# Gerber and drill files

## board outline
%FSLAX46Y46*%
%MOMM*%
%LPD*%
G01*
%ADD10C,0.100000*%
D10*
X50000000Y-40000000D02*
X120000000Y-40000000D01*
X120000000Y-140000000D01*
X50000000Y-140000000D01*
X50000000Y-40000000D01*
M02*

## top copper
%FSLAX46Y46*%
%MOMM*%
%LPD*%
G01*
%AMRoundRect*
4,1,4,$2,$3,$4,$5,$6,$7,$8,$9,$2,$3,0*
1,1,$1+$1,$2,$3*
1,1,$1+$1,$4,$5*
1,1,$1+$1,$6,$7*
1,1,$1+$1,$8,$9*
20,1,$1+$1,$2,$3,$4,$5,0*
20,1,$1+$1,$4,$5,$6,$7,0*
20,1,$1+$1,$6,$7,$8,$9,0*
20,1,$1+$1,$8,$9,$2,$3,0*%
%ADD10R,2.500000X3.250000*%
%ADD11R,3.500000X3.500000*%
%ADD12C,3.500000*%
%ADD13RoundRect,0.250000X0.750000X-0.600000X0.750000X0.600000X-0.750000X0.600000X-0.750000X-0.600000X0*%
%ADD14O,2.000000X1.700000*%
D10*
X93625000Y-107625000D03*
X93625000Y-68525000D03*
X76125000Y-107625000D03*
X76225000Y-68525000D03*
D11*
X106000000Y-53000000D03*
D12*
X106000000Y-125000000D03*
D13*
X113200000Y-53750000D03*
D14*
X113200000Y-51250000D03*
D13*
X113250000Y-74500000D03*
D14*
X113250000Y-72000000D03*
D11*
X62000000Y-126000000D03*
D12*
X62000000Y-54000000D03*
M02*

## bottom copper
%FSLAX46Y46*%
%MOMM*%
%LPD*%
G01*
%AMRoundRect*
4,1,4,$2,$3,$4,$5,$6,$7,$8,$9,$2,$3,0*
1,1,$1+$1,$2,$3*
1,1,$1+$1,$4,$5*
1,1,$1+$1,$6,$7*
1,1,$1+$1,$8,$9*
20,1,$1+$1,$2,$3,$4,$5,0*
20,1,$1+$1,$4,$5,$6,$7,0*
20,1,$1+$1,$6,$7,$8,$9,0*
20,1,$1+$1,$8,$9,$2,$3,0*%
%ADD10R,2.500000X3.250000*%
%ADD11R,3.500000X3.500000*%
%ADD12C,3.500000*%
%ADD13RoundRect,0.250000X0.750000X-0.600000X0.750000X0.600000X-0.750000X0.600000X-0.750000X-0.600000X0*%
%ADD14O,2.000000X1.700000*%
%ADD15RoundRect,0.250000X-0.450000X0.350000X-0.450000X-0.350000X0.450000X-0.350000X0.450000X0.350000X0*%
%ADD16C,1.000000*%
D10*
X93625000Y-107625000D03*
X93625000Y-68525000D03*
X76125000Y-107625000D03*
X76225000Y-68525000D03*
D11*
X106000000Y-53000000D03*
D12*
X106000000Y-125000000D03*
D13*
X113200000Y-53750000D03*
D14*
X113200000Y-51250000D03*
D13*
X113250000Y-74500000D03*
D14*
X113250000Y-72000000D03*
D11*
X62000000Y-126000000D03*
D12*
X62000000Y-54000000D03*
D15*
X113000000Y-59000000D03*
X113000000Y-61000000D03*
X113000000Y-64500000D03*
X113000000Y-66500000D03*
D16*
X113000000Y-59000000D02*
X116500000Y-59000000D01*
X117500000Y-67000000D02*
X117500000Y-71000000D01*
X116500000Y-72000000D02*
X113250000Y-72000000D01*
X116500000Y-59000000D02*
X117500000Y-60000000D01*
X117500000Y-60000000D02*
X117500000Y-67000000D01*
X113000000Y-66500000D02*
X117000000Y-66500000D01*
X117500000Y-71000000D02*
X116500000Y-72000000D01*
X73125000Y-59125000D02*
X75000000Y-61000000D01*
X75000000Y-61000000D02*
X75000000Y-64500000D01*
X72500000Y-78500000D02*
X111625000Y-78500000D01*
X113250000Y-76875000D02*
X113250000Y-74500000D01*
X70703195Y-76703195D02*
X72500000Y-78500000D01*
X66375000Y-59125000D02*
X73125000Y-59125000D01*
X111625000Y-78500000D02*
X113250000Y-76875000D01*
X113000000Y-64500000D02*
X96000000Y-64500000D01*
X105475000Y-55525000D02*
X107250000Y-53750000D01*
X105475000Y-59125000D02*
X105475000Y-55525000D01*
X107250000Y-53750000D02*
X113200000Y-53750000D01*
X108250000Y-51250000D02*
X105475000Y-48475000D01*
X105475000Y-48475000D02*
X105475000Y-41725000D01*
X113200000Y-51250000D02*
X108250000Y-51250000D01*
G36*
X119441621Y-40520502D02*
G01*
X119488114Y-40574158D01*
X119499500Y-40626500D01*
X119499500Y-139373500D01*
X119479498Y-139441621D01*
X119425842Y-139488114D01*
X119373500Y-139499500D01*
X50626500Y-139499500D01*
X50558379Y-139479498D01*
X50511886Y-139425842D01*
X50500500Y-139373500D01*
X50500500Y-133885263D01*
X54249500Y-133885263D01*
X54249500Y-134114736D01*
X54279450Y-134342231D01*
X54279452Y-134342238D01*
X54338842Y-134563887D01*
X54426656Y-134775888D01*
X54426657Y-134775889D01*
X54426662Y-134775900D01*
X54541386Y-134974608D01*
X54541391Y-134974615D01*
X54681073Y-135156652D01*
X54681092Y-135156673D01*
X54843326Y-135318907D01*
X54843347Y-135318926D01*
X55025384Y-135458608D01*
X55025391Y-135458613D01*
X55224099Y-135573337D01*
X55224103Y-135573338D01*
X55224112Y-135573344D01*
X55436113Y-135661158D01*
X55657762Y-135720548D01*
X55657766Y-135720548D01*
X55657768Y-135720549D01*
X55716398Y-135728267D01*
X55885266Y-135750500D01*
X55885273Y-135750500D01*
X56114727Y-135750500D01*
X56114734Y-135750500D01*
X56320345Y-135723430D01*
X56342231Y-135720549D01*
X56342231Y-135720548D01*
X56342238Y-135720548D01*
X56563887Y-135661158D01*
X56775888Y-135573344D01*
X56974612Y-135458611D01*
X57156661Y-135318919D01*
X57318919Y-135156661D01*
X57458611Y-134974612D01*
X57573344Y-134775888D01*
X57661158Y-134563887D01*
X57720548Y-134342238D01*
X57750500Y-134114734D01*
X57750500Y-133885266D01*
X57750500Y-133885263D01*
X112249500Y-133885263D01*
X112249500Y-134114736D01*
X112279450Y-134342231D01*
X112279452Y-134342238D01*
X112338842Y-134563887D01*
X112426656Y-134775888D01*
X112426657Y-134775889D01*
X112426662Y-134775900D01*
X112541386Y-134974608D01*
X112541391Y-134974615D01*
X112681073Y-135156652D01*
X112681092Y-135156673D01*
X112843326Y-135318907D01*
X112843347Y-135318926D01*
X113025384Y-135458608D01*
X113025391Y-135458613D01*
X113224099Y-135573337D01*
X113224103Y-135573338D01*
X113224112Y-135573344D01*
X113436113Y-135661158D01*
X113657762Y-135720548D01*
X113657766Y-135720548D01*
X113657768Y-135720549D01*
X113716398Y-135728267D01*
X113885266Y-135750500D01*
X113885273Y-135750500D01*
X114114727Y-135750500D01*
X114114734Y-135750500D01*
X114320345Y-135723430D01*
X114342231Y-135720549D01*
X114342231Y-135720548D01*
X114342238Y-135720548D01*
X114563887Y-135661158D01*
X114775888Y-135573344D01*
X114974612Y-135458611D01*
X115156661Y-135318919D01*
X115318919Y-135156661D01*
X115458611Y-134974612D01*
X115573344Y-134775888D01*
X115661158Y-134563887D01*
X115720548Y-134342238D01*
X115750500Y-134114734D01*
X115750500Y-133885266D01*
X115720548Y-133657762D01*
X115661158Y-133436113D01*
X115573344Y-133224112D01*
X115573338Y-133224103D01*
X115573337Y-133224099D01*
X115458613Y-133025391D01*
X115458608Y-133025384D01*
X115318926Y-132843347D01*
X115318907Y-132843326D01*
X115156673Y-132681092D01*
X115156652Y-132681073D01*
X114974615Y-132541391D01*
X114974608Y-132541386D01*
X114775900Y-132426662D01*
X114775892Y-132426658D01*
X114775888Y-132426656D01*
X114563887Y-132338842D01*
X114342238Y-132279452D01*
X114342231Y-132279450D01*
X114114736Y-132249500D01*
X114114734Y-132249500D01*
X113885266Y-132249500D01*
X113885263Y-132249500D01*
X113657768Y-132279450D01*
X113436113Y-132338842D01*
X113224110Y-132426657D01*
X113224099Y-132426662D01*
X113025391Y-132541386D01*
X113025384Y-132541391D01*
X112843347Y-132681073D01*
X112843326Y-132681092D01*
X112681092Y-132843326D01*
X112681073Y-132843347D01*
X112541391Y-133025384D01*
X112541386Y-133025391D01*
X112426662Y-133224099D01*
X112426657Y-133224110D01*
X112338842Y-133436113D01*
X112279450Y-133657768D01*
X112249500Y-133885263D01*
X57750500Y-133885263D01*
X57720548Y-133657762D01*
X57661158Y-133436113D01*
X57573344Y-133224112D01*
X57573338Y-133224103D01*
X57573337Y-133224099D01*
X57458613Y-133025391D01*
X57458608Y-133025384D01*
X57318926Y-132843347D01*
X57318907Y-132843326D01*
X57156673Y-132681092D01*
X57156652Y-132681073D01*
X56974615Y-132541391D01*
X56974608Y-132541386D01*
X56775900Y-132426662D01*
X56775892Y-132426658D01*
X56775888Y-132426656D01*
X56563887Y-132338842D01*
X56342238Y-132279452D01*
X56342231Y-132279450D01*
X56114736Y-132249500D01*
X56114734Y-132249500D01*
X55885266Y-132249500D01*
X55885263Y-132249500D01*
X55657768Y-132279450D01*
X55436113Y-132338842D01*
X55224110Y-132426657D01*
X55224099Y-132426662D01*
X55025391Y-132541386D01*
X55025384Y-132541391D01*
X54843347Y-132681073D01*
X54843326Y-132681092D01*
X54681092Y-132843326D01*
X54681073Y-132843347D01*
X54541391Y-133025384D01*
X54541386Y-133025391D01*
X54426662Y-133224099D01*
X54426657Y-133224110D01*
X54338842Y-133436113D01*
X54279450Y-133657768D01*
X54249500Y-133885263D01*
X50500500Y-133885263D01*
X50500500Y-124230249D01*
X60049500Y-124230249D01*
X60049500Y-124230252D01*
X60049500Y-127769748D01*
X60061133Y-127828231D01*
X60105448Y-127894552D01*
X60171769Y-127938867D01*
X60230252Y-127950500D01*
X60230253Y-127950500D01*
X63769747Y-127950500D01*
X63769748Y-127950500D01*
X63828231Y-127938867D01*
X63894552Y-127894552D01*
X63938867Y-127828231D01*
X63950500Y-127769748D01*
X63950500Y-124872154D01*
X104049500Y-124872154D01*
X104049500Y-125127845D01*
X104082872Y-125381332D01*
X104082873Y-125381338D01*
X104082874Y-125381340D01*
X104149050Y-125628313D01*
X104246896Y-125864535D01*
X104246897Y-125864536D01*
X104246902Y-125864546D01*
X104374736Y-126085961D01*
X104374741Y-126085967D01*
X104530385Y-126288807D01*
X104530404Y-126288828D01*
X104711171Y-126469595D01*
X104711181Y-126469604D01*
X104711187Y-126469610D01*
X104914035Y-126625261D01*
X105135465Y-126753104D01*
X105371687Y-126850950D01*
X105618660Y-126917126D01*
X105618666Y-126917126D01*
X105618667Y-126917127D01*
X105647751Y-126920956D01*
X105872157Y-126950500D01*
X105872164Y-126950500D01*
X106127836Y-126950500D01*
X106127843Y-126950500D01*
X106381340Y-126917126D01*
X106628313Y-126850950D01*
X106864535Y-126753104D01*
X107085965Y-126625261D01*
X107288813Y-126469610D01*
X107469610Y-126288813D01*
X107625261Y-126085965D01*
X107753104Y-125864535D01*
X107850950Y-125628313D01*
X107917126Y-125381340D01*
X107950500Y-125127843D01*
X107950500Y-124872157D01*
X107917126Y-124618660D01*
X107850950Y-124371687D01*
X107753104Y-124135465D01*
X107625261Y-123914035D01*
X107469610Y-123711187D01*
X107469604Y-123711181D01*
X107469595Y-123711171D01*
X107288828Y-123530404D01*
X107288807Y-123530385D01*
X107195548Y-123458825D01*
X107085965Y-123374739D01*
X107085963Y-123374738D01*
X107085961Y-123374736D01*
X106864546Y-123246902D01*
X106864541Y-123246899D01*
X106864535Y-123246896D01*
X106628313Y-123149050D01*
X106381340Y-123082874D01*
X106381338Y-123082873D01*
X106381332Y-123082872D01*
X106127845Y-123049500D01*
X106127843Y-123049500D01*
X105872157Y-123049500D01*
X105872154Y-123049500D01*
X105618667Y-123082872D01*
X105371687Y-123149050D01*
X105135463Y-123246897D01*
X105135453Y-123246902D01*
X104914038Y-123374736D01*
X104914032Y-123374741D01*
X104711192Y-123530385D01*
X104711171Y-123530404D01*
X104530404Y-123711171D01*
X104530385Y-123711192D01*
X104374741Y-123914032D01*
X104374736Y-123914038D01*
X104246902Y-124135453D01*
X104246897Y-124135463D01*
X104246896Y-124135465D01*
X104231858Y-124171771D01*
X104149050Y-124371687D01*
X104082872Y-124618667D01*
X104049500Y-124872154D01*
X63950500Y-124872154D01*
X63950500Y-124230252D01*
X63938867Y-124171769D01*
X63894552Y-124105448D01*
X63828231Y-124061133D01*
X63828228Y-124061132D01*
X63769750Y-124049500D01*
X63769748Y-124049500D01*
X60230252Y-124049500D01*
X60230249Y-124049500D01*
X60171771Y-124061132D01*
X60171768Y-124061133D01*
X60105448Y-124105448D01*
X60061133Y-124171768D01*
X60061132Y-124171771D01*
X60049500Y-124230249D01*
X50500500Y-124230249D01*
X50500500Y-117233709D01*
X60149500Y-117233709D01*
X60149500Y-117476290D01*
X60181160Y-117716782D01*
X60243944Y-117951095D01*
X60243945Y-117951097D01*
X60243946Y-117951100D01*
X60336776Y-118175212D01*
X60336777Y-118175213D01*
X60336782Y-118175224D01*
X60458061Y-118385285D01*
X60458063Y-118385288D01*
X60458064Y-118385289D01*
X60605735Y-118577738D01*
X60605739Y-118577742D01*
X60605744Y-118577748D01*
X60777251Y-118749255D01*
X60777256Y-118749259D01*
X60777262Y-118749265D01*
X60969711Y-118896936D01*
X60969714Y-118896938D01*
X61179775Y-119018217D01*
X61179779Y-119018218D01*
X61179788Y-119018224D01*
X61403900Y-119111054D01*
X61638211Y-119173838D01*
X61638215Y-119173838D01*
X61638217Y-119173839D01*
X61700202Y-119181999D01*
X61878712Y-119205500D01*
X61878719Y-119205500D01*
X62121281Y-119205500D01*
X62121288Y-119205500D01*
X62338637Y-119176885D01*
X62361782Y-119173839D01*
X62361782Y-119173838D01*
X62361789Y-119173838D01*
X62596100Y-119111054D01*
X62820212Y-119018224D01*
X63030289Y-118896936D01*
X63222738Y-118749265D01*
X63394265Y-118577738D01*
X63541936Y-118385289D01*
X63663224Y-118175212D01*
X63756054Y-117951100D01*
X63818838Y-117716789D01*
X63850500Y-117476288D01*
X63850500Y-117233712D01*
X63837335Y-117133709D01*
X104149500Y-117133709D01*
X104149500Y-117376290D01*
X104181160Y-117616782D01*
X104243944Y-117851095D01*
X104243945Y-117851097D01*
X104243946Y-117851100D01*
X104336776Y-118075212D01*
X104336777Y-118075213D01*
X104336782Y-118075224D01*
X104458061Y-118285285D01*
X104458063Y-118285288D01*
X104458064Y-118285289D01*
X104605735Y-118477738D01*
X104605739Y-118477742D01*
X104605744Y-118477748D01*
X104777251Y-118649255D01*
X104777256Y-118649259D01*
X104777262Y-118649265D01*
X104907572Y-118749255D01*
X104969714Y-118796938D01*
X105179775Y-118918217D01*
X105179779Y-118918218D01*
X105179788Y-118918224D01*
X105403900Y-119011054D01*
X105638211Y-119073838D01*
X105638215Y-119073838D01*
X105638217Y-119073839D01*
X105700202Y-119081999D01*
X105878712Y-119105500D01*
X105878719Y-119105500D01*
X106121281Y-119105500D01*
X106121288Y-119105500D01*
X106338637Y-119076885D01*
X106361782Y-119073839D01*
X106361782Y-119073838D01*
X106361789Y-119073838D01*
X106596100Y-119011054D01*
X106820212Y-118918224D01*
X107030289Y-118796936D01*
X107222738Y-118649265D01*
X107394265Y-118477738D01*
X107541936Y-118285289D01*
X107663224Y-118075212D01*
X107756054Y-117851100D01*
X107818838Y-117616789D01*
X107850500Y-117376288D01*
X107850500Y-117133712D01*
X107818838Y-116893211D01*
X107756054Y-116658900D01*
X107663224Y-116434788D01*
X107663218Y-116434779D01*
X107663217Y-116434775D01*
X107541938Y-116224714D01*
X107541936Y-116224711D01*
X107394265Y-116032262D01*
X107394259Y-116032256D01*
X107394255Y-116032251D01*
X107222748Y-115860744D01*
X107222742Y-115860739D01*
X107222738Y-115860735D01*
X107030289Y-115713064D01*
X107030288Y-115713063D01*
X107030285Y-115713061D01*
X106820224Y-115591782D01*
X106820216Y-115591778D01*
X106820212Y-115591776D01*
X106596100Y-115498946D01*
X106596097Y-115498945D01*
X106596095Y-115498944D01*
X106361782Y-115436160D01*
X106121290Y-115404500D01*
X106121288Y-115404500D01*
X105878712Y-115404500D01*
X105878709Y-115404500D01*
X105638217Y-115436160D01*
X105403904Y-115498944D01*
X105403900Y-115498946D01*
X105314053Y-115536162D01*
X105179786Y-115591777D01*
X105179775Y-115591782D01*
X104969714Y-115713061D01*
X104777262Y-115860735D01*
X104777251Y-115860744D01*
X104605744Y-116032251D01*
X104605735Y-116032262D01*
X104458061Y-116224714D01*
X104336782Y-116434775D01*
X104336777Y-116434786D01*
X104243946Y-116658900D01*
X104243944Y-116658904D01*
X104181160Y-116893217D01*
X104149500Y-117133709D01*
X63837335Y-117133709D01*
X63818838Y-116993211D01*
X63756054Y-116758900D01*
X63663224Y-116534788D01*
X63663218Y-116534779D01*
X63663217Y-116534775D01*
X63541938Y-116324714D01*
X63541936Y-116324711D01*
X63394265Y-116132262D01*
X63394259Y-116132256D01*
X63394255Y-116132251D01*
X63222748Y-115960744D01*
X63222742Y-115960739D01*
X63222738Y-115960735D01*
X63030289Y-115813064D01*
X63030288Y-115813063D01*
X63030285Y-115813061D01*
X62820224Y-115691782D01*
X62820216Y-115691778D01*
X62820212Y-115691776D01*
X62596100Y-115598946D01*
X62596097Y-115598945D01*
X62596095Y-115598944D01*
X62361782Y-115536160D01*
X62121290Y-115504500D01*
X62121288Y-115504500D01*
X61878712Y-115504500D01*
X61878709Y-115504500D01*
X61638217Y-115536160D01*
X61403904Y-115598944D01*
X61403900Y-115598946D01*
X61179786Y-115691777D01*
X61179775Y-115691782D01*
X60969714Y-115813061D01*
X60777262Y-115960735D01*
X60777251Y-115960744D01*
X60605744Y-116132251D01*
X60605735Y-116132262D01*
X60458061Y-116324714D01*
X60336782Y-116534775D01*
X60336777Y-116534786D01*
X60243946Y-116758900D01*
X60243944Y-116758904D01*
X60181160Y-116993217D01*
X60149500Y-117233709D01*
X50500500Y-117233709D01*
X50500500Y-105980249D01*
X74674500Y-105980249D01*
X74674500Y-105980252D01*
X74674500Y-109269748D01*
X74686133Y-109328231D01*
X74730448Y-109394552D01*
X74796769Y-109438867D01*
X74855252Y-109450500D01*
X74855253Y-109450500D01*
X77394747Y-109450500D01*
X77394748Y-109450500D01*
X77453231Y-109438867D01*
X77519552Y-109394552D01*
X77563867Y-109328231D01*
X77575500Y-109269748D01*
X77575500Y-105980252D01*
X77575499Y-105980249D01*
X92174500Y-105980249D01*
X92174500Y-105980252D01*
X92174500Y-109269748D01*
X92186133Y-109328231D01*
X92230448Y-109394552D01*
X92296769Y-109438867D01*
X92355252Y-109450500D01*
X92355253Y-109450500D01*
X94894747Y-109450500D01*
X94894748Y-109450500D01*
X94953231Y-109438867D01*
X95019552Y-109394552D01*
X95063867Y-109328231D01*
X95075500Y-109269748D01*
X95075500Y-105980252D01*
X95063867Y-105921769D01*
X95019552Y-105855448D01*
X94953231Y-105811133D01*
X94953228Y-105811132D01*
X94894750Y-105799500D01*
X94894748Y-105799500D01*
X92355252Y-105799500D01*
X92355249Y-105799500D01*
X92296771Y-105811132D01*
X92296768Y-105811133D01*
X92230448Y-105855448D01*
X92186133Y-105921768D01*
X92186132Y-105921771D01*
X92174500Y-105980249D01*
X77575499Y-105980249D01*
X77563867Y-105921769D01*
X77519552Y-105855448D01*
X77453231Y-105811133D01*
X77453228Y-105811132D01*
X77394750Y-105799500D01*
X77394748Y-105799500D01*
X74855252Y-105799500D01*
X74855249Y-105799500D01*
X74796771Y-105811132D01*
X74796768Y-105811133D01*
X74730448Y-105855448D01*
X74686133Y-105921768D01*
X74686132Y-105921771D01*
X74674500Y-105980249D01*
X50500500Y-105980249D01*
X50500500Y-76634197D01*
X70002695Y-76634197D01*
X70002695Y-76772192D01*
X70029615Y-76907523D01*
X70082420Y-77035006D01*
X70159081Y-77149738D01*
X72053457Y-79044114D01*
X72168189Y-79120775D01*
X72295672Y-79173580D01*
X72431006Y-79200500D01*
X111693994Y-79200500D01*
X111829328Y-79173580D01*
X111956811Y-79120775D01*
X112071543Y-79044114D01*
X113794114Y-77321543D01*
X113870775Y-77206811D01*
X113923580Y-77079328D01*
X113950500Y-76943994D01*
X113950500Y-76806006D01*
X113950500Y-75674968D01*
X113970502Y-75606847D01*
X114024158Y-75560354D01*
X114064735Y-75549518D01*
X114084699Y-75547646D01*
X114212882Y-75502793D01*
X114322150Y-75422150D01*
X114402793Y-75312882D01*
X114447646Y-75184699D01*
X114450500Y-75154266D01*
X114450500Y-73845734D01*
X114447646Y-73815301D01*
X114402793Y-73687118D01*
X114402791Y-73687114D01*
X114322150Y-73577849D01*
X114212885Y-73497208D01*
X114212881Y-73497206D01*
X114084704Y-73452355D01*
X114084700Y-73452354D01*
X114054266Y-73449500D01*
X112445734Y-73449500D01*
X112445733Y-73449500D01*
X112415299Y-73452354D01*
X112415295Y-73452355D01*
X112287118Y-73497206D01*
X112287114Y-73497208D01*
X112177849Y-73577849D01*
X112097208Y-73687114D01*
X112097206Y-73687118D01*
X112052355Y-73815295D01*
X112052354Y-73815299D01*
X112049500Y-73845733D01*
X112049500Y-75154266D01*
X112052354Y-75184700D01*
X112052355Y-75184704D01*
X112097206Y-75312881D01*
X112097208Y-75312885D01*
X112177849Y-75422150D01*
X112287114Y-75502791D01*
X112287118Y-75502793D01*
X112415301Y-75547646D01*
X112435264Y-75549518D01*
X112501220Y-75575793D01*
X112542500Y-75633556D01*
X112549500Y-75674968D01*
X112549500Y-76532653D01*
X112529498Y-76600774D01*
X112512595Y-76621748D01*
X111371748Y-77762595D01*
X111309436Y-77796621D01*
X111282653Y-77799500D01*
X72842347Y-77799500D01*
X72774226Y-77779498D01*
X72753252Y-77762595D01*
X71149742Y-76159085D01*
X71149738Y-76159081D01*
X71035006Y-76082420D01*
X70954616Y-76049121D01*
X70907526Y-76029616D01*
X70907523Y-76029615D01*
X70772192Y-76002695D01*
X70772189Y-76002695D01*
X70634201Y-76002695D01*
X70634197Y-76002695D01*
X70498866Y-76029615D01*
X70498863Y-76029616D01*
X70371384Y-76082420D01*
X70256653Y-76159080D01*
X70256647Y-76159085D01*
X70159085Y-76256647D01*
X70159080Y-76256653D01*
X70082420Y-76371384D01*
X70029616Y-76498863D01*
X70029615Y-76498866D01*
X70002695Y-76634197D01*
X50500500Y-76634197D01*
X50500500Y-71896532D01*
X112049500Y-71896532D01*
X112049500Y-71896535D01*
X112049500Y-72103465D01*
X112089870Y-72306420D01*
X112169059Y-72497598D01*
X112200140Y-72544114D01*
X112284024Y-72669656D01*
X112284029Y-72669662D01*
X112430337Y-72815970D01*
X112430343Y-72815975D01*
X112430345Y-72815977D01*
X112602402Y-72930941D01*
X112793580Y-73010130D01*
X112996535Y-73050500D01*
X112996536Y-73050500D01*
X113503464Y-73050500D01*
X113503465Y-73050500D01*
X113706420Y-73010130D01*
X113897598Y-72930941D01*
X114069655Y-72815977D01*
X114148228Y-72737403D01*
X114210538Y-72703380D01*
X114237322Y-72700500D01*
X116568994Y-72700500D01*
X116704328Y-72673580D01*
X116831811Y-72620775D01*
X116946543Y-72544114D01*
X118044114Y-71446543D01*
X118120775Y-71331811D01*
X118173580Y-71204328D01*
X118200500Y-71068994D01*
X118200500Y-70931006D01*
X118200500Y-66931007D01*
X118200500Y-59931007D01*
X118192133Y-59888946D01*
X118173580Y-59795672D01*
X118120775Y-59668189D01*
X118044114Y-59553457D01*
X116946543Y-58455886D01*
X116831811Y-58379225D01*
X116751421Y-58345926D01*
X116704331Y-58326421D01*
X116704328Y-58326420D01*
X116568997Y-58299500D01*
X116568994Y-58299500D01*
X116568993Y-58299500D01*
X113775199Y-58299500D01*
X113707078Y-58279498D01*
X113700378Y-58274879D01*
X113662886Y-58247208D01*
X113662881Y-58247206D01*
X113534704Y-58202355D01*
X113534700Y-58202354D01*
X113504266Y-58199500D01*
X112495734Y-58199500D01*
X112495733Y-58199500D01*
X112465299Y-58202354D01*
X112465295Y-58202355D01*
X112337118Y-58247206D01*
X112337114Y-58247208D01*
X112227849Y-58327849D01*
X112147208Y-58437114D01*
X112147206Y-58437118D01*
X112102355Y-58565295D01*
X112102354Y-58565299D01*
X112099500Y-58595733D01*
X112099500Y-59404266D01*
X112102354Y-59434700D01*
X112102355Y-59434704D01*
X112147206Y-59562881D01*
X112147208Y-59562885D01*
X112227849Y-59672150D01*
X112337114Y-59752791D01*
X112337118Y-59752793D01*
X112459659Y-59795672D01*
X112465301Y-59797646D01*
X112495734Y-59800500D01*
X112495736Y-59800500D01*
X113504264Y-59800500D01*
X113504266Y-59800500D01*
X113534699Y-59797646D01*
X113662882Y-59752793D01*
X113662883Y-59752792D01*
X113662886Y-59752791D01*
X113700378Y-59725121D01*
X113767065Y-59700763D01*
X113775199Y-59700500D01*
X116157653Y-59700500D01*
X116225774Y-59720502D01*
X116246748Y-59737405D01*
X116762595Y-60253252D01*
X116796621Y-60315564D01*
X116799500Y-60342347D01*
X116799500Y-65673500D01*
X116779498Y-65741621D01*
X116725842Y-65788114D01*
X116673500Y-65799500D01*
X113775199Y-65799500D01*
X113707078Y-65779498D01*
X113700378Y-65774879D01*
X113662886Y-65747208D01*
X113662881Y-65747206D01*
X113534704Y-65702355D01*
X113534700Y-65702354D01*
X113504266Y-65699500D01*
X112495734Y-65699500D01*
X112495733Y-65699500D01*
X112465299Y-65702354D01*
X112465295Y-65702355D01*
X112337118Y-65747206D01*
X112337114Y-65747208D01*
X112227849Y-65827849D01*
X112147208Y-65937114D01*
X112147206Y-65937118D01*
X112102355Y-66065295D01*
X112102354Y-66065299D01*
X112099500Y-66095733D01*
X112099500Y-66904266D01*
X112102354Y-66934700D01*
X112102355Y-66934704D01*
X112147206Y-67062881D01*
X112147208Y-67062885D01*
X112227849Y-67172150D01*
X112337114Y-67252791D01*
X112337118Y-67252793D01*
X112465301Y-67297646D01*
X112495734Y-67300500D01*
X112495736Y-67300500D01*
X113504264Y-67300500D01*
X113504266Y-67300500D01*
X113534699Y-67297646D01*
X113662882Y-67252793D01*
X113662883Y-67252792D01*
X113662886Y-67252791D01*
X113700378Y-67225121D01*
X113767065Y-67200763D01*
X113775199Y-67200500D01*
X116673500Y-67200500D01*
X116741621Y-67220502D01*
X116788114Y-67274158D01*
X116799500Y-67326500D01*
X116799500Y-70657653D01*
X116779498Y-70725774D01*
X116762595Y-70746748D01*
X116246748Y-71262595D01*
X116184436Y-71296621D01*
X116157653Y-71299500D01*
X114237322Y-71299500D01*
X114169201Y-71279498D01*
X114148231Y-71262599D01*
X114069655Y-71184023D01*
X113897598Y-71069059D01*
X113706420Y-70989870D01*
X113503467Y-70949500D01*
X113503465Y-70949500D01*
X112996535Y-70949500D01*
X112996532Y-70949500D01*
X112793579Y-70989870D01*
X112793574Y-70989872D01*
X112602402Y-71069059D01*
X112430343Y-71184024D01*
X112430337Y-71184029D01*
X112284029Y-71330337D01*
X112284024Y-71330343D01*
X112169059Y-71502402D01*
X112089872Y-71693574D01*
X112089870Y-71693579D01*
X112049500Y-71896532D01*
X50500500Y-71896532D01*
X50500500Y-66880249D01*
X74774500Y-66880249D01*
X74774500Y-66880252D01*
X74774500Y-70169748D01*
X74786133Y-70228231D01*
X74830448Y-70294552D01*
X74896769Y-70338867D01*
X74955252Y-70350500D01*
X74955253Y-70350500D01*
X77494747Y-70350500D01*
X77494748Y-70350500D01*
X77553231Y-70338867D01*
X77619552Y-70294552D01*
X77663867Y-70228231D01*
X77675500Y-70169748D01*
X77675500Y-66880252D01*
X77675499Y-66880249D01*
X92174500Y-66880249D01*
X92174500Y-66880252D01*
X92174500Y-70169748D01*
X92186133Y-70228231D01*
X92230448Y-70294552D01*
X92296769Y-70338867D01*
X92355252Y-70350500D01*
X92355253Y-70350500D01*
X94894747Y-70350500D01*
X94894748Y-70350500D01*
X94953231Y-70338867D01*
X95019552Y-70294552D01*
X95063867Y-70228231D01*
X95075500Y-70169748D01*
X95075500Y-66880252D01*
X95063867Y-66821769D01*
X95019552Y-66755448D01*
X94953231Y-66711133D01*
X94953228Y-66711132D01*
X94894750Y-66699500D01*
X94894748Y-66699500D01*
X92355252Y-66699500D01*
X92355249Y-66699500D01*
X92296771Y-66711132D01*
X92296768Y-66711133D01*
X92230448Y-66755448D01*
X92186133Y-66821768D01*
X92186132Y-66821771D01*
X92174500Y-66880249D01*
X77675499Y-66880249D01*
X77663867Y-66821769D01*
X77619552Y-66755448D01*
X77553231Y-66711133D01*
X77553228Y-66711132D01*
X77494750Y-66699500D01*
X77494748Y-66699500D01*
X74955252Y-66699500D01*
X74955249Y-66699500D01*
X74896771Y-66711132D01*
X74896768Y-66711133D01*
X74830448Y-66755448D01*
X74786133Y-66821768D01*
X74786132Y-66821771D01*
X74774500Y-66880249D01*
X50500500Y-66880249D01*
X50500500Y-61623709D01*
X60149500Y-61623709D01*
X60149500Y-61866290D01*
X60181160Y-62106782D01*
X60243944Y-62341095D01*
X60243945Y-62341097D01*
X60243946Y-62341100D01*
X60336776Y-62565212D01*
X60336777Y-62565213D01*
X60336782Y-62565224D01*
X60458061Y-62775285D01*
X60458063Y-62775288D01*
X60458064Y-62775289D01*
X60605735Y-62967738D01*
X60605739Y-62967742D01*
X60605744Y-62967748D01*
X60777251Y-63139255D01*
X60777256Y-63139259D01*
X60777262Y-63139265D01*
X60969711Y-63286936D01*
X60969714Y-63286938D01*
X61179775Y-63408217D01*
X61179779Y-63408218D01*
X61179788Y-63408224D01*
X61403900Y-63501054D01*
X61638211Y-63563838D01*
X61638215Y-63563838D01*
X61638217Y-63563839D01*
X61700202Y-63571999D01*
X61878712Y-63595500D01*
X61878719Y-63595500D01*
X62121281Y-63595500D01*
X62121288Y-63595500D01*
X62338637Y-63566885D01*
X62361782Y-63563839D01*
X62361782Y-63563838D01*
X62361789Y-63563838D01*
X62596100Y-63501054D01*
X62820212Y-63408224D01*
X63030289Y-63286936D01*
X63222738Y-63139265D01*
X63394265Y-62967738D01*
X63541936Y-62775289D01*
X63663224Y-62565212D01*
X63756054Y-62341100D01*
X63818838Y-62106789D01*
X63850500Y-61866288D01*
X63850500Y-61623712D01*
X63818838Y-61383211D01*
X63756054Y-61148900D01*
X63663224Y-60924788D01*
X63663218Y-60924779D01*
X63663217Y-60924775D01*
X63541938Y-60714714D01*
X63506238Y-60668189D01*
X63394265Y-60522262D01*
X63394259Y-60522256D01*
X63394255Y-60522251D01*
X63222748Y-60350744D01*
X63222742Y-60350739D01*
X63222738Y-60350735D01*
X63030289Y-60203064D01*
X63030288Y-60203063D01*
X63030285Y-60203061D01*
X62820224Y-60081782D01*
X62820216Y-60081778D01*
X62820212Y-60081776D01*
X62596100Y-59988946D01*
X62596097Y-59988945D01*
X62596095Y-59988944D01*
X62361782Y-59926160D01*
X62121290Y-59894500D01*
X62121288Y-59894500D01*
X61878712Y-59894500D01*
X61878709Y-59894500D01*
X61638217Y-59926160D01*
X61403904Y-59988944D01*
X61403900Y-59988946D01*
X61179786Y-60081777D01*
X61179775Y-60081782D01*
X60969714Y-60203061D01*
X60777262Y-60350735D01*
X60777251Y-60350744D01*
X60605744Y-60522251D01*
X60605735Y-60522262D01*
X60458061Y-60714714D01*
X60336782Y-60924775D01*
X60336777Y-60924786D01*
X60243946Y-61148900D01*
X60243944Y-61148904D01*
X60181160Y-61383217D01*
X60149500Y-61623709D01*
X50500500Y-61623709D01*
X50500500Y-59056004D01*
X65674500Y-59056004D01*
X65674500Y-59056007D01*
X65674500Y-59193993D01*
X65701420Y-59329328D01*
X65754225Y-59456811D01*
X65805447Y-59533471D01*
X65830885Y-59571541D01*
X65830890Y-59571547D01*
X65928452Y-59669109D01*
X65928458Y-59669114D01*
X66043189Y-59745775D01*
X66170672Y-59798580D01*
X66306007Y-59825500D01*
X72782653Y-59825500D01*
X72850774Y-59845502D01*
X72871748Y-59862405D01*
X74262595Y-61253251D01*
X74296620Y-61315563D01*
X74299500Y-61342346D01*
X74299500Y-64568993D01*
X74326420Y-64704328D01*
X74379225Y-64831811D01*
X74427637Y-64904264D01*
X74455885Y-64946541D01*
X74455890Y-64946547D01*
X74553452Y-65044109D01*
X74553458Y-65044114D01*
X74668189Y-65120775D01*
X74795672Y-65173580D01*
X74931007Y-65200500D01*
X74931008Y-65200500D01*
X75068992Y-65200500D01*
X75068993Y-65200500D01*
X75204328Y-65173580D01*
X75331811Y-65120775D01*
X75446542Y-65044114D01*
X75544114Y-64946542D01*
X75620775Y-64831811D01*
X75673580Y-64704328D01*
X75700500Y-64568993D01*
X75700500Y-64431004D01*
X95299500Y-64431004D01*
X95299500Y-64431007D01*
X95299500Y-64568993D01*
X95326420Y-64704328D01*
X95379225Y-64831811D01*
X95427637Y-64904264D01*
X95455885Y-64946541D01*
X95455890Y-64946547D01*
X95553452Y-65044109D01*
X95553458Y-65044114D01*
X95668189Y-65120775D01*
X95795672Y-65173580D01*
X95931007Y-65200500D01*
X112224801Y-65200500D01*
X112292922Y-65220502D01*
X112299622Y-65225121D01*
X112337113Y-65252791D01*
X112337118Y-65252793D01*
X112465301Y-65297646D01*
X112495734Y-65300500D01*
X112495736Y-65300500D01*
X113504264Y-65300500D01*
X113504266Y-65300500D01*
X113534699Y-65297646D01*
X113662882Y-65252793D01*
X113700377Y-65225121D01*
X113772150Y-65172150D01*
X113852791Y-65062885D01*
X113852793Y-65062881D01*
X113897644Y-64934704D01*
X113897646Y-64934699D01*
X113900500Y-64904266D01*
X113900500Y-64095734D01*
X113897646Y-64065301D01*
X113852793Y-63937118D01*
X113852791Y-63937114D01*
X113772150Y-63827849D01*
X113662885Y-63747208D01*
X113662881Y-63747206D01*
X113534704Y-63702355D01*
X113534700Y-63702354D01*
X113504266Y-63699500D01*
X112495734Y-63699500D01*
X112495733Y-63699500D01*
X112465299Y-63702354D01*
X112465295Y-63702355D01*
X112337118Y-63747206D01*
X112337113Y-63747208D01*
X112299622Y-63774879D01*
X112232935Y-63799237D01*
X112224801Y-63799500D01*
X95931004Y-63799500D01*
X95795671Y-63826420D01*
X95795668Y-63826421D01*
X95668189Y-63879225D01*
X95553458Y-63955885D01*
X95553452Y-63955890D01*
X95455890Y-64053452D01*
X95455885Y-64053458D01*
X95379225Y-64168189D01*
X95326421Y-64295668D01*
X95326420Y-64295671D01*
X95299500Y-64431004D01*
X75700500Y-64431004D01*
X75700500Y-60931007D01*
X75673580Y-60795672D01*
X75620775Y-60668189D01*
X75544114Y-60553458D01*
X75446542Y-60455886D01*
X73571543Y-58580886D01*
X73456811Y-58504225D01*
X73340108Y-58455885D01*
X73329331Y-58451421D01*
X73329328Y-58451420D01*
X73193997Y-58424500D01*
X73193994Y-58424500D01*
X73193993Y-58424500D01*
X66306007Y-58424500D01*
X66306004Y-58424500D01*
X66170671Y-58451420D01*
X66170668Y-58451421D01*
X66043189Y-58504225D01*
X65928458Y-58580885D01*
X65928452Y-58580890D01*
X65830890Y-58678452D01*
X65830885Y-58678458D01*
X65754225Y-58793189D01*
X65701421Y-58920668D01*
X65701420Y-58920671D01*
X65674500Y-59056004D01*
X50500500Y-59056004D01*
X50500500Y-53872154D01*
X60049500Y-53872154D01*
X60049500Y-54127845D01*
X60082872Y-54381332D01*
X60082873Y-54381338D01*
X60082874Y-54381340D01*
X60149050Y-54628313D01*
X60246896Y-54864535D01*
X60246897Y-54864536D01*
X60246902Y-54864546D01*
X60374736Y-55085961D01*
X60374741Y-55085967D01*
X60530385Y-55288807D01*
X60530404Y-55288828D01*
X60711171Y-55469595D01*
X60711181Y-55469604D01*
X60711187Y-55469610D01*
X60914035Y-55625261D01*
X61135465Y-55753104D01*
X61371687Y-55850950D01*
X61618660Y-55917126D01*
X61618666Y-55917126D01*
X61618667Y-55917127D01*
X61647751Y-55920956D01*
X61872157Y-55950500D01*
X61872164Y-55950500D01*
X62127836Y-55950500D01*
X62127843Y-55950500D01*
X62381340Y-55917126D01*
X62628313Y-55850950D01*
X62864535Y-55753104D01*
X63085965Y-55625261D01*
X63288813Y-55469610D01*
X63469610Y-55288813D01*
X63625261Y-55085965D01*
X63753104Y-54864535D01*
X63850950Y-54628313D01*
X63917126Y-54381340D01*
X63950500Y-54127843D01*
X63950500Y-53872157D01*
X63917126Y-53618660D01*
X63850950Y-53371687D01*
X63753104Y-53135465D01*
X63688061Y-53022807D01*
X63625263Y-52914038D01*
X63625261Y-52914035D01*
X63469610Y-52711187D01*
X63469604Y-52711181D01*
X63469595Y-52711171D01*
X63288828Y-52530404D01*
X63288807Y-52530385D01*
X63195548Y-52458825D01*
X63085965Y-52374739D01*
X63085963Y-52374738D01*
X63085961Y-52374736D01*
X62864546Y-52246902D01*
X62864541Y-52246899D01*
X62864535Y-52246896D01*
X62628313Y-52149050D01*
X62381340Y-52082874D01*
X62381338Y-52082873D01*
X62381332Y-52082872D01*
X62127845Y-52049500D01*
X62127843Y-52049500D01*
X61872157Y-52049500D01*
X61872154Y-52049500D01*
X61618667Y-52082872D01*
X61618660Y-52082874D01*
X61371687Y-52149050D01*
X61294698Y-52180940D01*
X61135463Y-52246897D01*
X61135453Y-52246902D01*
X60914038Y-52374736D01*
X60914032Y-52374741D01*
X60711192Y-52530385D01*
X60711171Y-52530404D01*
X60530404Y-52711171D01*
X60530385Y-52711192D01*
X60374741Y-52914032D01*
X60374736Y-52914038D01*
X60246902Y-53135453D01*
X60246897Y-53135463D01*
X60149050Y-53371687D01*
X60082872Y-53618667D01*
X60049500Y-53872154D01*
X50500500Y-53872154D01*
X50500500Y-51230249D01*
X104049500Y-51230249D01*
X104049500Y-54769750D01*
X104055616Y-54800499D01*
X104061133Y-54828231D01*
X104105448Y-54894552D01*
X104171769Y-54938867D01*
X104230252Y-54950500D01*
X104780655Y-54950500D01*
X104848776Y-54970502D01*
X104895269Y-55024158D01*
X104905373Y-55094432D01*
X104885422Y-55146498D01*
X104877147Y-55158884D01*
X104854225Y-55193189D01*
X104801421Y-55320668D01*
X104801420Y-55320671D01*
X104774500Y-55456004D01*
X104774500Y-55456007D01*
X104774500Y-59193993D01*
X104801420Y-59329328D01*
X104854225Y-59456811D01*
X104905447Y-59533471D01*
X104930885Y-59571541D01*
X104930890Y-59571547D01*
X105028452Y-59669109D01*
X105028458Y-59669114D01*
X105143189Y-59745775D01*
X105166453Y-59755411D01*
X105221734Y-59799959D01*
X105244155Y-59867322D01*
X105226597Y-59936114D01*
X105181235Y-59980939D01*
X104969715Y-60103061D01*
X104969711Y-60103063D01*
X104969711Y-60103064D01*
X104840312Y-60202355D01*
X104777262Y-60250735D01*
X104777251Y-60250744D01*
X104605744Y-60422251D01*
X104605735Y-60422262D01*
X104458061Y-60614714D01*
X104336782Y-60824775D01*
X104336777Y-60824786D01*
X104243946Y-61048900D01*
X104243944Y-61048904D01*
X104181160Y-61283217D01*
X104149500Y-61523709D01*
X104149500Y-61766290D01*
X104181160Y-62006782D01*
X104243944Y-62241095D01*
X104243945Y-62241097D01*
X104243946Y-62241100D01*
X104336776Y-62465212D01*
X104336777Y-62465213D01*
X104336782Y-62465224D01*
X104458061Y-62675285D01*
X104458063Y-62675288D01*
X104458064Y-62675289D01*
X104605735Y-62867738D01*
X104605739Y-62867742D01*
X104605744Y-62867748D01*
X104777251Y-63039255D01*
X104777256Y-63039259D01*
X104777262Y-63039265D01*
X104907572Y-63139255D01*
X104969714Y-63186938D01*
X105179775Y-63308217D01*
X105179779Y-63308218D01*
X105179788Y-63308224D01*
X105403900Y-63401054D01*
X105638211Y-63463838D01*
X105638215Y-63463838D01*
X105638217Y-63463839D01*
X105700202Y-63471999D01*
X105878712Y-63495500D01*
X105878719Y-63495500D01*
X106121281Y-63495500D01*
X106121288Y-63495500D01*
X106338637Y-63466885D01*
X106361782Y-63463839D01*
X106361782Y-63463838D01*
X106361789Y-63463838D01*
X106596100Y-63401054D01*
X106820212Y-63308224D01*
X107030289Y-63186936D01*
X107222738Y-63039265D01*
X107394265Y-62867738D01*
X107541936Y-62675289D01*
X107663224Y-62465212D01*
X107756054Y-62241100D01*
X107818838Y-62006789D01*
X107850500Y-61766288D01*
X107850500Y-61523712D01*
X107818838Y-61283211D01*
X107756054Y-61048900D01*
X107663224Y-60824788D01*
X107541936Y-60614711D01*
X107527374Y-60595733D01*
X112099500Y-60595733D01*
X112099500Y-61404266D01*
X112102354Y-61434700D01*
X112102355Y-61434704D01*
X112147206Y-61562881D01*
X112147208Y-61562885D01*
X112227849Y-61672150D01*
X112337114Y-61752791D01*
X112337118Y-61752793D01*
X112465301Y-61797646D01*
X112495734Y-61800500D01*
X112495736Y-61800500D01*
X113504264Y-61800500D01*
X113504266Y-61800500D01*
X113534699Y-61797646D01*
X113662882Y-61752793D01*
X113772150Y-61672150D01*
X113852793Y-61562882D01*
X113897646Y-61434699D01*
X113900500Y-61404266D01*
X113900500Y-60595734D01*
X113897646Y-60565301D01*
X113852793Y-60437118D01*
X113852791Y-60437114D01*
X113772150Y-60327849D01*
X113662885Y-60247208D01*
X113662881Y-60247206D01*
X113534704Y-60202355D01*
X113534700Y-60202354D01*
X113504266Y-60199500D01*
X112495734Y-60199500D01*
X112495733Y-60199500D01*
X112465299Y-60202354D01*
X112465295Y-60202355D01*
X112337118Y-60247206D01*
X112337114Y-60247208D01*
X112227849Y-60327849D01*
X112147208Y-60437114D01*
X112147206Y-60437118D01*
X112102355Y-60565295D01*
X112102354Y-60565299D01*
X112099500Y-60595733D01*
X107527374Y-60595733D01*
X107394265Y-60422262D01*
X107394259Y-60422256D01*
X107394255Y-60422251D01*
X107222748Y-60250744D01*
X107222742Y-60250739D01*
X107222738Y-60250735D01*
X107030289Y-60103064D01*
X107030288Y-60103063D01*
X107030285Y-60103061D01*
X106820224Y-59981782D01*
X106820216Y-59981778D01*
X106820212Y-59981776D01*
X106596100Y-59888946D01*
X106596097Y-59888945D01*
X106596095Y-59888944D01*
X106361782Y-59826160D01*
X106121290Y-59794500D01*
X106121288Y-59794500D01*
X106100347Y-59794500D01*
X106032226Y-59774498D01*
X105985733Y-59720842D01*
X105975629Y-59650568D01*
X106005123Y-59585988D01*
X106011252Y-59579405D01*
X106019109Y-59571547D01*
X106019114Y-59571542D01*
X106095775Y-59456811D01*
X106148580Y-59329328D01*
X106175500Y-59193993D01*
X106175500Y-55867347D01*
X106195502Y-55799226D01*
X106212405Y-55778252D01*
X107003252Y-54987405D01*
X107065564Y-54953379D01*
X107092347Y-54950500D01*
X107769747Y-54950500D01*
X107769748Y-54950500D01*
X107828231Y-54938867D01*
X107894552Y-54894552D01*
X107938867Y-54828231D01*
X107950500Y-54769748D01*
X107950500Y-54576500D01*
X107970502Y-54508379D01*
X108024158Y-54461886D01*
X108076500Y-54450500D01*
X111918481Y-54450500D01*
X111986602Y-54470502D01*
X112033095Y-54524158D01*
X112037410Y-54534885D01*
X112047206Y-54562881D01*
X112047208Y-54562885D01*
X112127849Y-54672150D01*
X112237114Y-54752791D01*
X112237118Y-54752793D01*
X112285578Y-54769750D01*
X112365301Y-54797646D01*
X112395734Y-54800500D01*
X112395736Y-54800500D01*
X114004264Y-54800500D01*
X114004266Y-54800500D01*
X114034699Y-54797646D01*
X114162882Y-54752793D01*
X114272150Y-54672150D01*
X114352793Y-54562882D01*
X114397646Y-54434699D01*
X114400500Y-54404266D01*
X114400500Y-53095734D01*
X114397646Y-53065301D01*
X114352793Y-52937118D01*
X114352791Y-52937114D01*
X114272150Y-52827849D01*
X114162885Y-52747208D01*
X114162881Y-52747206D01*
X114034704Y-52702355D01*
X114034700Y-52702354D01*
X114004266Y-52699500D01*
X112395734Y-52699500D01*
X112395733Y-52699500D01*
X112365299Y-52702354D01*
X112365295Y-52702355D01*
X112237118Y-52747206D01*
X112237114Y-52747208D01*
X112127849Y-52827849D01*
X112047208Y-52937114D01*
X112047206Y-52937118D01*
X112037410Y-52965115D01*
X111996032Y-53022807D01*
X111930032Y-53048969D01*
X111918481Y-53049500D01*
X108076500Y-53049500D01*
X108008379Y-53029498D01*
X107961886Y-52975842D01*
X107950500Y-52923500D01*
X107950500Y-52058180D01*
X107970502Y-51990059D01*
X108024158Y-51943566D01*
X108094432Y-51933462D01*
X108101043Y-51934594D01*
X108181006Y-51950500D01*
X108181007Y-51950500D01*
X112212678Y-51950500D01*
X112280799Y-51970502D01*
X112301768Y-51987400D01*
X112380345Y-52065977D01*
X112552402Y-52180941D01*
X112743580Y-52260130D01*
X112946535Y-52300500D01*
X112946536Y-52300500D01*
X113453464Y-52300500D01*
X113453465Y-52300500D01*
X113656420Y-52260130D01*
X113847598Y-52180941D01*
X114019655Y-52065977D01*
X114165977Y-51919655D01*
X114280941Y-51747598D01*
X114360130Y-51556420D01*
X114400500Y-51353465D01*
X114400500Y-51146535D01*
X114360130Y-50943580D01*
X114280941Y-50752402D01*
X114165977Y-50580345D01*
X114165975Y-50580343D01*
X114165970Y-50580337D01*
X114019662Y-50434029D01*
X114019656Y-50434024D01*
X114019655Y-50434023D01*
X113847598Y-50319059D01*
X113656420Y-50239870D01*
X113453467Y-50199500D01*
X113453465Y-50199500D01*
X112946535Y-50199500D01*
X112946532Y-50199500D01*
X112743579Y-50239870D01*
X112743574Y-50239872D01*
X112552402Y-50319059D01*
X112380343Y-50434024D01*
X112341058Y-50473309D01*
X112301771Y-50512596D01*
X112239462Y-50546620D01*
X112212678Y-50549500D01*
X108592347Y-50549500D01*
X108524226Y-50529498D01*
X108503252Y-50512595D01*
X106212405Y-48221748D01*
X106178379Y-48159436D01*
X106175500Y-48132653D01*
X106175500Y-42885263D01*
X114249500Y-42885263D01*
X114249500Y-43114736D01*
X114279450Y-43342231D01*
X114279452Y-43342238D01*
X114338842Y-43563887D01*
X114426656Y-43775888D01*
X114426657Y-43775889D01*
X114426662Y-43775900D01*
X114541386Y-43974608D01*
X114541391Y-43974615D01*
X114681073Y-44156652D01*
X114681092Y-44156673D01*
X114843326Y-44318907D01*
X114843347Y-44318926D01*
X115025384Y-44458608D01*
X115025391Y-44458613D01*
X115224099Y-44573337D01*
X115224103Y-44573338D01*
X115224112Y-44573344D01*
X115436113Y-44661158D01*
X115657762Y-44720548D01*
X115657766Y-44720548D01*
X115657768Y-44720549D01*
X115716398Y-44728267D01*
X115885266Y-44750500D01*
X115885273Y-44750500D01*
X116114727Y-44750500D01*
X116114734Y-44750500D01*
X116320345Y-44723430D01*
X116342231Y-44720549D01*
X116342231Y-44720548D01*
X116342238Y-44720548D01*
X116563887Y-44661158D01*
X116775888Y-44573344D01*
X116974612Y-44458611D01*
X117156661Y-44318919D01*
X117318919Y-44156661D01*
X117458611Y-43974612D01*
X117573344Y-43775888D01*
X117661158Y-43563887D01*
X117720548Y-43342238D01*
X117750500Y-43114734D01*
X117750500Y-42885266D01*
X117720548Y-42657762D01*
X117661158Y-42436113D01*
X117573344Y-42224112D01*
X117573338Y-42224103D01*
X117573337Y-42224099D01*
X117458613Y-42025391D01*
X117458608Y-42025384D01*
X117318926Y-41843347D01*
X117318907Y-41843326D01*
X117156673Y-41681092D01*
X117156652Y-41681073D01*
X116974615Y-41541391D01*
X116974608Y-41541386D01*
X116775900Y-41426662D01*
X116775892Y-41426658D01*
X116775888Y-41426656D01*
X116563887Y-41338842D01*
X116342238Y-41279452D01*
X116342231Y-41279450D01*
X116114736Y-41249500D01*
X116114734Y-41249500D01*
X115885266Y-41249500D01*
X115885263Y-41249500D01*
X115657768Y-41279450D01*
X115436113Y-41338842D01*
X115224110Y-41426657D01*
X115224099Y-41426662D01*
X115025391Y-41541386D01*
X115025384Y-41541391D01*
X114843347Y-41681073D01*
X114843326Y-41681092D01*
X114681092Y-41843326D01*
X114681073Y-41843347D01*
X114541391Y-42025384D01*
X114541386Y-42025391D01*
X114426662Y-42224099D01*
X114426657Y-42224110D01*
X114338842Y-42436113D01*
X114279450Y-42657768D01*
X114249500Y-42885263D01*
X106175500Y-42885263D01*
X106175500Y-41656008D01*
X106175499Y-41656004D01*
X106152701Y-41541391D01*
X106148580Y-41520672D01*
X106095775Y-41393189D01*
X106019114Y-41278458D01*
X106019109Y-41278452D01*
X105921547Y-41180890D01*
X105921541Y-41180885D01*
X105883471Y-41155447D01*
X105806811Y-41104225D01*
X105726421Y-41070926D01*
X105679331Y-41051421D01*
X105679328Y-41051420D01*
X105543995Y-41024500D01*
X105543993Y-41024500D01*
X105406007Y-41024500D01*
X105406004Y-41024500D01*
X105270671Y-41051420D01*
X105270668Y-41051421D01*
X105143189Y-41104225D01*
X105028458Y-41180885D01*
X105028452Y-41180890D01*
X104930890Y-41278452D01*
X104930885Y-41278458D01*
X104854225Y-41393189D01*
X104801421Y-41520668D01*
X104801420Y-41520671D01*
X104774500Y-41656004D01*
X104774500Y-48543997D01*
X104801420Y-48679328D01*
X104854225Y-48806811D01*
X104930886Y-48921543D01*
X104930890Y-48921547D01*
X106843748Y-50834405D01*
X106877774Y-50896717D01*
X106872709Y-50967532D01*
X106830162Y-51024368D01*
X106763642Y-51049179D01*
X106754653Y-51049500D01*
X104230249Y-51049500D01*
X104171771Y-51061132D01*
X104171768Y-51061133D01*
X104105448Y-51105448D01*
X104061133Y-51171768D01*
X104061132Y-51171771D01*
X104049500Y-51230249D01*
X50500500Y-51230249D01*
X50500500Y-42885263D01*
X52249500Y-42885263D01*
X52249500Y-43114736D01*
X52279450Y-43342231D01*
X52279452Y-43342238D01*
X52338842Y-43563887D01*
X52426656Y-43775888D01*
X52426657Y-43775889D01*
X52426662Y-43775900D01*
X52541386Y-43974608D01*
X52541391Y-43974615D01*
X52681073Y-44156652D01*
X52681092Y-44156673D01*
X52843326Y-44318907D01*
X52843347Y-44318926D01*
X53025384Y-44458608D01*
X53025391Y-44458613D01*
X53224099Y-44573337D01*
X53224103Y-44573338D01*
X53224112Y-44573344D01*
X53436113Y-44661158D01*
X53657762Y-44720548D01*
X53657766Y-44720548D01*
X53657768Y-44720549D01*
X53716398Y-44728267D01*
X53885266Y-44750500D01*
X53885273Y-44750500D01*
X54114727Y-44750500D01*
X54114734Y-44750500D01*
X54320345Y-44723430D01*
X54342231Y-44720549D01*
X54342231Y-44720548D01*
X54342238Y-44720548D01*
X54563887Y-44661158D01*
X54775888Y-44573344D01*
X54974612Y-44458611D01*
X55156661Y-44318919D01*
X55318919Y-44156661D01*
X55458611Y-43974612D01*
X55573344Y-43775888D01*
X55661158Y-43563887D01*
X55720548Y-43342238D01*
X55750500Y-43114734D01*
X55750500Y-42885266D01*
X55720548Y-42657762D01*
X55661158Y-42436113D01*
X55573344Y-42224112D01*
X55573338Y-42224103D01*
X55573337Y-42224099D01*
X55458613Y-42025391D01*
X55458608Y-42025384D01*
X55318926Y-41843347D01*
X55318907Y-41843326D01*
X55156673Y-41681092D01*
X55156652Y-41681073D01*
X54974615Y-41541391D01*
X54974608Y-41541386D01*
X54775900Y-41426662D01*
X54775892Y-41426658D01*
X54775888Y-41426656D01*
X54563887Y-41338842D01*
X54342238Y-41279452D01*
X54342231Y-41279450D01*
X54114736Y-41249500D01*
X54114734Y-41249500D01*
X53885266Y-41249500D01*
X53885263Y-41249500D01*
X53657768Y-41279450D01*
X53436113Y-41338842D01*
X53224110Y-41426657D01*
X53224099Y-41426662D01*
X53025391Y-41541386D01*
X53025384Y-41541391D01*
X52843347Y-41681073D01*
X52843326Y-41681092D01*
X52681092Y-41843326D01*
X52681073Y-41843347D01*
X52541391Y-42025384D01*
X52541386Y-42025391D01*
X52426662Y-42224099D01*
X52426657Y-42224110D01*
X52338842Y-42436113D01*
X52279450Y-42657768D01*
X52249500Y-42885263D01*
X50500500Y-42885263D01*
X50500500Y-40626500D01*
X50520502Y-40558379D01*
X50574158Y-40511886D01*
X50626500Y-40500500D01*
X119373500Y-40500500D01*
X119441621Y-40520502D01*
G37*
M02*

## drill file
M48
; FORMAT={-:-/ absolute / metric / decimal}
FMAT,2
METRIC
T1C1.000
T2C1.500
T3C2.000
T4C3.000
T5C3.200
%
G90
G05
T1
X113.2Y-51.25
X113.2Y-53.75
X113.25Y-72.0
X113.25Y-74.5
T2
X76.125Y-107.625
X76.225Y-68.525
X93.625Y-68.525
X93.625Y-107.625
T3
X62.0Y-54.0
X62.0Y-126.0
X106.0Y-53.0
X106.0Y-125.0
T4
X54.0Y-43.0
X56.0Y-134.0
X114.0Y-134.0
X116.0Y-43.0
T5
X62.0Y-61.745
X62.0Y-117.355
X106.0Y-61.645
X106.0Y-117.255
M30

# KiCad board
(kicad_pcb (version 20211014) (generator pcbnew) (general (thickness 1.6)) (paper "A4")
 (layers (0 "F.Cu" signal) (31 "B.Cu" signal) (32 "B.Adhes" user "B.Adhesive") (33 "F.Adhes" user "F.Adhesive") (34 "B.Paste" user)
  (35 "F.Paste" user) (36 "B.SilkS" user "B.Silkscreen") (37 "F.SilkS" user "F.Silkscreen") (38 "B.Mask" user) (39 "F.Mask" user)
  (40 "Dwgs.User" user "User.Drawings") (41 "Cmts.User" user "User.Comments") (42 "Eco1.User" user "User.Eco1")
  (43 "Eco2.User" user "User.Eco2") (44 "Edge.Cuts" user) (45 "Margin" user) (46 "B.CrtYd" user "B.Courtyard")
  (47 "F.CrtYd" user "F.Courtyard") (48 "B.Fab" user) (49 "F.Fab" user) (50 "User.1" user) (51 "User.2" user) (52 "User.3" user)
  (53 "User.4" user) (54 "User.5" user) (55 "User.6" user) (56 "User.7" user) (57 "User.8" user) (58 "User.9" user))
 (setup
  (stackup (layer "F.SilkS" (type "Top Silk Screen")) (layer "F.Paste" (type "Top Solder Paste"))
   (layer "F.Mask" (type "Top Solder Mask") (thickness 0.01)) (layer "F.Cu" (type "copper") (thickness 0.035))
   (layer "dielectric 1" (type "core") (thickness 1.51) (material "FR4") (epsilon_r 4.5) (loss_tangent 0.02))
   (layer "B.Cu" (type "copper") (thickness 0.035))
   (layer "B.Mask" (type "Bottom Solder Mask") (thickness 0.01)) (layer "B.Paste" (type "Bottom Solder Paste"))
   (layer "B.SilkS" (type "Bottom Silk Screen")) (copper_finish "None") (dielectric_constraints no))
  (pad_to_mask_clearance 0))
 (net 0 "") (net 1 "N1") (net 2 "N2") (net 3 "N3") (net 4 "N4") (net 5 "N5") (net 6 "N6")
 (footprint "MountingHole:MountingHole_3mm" (layer "F.Cu") (at 54 43)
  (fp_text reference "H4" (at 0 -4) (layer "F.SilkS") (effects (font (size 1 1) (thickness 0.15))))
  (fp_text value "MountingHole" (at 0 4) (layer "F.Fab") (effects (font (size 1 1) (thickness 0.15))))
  (pad "" np_thru_hole circle (at 0 0) (size 3 3) (drill 3) (layers *.Cu *.Mask)))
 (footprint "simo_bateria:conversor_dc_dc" (layer "F.Cu") (at 93.625 107.625 180)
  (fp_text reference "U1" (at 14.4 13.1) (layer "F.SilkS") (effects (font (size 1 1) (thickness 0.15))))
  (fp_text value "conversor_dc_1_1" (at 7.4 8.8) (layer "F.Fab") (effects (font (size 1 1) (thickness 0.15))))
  (pad "1" thru_hole rect (at 0 0 180) (size 2.5 3.25) (drill 1.5) (layers *.Cu *.Mask) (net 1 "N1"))
  (pad "2" thru_hole rect (at 0 39.1 180) (size 2.5 3.25) (drill 1.5) (layers *.Cu *.Mask) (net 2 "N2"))
  (pad "3" thru_hole rect (at 17.5 0 180) (size 2.5 3.25) (drill 1.5) (layers *.Cu *.Mask) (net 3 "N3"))
  (pad "4" thru_hole rect (at 17.4 39.1 180) (size 2.5 3.25) (drill 1.5) (layers *.Cu *.Mask) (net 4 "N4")))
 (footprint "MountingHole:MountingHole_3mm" (layer "F.Cu") (at 116 43)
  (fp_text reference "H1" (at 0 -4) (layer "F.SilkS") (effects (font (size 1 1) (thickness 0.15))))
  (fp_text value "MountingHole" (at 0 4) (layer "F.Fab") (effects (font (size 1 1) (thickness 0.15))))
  (pad "" np_thru_hole circle (at 0 0) (size 3 3) (drill 3) (layers *.Cu *.Mask)))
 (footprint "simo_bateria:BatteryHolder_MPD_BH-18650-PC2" (layer "F.Cu") (at 106 53 -90)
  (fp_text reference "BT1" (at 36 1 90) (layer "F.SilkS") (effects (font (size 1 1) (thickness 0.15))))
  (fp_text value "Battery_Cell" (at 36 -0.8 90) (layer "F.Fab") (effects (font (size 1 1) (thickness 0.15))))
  (pad "" np_thru_hole circle (at 8.645 0 270) (size 3.2 3.2) (drill 3.2) (layers *.Cu *.Mask))
  (pad "" np_thru_hole circle (at 64.255 0 270) (size 3.2 3.2) (drill 3.2) (layers *.Cu *.Mask))
  (pad "1" thru_hole rect (at 0 0 270) (size 3.5 3.5) (drill 2) (layers *.Cu *.Mask) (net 3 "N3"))
  (pad "2" thru_hole circle (at 72 0 270) (size 3.5 3.5) (drill 2) (layers *.Cu *.Mask) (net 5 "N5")))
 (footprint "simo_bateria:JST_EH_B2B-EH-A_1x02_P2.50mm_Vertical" (layer "F.Cu") (at 113.2 53.75 90)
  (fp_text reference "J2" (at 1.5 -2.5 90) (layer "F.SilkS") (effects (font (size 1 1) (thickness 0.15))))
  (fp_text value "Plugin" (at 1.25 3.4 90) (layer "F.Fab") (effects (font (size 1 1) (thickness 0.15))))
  (pad "1" thru_hole roundrect (at 0 0 90) (size 1.7 2) (drill 1) (layers *.Cu *.Mask) (roundrect_rratio 0.147059) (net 2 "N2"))
  (pad "2" thru_hole oval (at 2.5 0 90) (size 1.7 2) (drill 1) (layers *.Cu *.Mask) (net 4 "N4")))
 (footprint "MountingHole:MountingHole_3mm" (layer "F.Cu") (at 56 134)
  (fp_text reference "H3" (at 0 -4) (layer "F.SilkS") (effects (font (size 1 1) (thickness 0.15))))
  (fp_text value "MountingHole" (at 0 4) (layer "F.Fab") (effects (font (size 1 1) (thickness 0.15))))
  (pad "" np_thru_hole circle (at 0 0) (size 3 3) (drill 3) (layers *.Cu *.Mask)))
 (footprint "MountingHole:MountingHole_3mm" (layer "F.Cu") (at 114 134)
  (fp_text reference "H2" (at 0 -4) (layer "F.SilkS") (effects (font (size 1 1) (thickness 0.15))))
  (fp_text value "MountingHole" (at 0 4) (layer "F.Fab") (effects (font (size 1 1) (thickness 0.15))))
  (pad "" np_thru_hole circle (at 0 0) (size 3 3) (drill 3) (layers *.Cu *.Mask)))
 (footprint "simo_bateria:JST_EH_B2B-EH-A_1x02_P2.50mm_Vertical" (layer "F.Cu") (at 113.25 74.5 90)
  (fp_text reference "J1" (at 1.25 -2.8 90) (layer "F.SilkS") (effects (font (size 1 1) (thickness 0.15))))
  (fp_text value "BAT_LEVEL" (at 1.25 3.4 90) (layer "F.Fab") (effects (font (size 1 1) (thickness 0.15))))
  (pad "1" thru_hole roundrect (at 0 0 90) (size 1.7 2) (drill 1) (layers *.Cu *.Mask) (roundrect_rratio 0.147059) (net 1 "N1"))
  (pad "2" thru_hole oval (at 2.5 0 90) (size 1.7 2) (drill 1) (layers *.Cu *.Mask) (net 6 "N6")))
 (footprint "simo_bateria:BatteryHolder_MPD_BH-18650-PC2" (layer "F.Cu") (at 62 126 90)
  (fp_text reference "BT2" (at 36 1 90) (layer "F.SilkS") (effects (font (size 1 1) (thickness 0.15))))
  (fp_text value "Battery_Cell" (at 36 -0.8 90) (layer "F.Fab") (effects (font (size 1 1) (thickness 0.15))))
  (pad "" np_thru_hole circle (at 64.255 0 90) (size 3.2 3.2) (drill 3.2) (layers *.Cu *.Mask))
  (pad "" np_thru_hole circle (at 8.645 0 90) (size 3.2 3.2) (drill 3.2) (layers *.Cu *.Mask))
  (pad "1" thru_hole rect (at 0 0 90) (size 3.5 3.5) (drill 2) (layers *.Cu *.Mask) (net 5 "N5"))
  (pad "2" thru_hole circle (at 72 0 90) (size 3.5 3.5) (drill 2) (layers *.Cu *.Mask) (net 1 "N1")))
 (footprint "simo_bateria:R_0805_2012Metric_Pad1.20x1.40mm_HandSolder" (layer "B.Cu") (at 113 60 -90)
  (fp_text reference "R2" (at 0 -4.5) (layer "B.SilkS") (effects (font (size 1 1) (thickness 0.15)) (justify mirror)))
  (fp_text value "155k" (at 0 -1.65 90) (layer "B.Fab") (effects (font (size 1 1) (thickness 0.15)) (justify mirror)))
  (pad "1" smd roundrect locked (at -1 0 270) (size 1.2 1.4) (layers "B.Cu" "B.Paste" "B.Mask") (roundrect_rratio 0.208333) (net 6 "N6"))
  (pad "2" smd roundrect locked (at 1 0 270) (size 1.2 1.4) (layers "B.Cu" "B.Paste" "B.Mask") (roundrect_rratio 0.208333) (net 1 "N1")))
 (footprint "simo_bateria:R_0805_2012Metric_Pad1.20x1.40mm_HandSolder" (layer "B.Cu") (at 113 65.5 -90)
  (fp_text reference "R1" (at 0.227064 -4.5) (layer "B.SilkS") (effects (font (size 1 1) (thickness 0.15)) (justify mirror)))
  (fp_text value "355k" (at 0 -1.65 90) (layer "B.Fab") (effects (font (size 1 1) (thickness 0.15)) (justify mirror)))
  (pad "1" smd roundrect locked (at -1 0 270) (size 1.2 1.4) (layers "B.Cu" "B.Paste" "B.Mask") (roundrect_rratio 0.208333) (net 3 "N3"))
  (pad "2" smd roundrect locked (at 1 0 270) (size 1.2 1.4) (layers "B.Cu" "B.Paste" "B.Mask") (roundrect_rratio 0.208333) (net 6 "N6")))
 (gr_rect (start 50 40) (end 120 140) (layer "Edge.Cuts") (width 0.1) (fill none))
 (segment (start 113 59) (end 116.5 59) (width 1) (layer "B.Cu") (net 6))
 (segment (start 117.5 67) (end 117.5 71) (width 1) (layer "B.Cu") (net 6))
 (segment (start 116.5 72) (end 113.25 72) (width 1) (layer "B.Cu") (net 6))
 (segment (start 116.5 59) (end 117.5 60) (width 1) (layer "B.Cu") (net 6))
 (segment (start 117.5 60) (end 117.5 67) (width 1) (layer "B.Cu") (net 6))
 (segment (start 113 66.5) (end 117 66.5) (width 1) (layer "B.Cu") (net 6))
 (segment (start 117.5 71) (end 116.5 72) (width 1) (layer "B.Cu") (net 6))
 (segment (start 73.125 59.125) (end 75 61) (width 1) (layer "B.Cu") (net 1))
 (segment (start 75 61) (end 75 64.5) (width 1) (layer "B.Cu") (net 1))
 (segment (start 72.5 78.5) (end 111.625 78.5) (width 1) (layer "B.Cu") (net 1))
 (segment (start 113.25 76.875) (end 113.25 74.5) (width 1) (layer "B.Cu") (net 1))
 (segment (start 70.703195 76.703195) (end 72.5 78.5) (width 1) (layer "B.Cu") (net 1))
 (segment (start 66.375 59.125) (end 73.125 59.125) (width 1) (layer "B.Cu") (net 1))
 (segment (start 111.625 78.5) (end 113.25 76.875) (width 1) (layer "B.Cu") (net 1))
 (segment (start 113 64.5) (end 96 64.5) (width 1) (layer "B.Cu") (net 3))
 (segment (start 105.475 55.525) (end 107.25 53.75) (width 1) (layer "B.Cu") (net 2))
 (segment (start 105.475 59.125) (end 105.475 55.525) (width 1) (layer "B.Cu") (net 2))
 (segment (start 107.25 53.75) (end 113.2 53.75) (width 1) (layer "B.Cu") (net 2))
 (segment (start 108.25 51.25) (end 105.475 48.475) (width 1) (layer "B.Cu") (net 4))
 (segment (start 105.475 48.475) (end 105.475 41.725) (width 1) (layer "B.Cu") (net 4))
 (segment (start 113.2 51.25) (end 108.25 51.25) (width 1) (layer "B.Cu") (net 4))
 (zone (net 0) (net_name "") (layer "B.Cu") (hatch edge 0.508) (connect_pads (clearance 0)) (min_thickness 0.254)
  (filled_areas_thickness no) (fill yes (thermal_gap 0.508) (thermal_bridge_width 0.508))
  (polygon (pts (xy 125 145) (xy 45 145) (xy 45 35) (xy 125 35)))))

